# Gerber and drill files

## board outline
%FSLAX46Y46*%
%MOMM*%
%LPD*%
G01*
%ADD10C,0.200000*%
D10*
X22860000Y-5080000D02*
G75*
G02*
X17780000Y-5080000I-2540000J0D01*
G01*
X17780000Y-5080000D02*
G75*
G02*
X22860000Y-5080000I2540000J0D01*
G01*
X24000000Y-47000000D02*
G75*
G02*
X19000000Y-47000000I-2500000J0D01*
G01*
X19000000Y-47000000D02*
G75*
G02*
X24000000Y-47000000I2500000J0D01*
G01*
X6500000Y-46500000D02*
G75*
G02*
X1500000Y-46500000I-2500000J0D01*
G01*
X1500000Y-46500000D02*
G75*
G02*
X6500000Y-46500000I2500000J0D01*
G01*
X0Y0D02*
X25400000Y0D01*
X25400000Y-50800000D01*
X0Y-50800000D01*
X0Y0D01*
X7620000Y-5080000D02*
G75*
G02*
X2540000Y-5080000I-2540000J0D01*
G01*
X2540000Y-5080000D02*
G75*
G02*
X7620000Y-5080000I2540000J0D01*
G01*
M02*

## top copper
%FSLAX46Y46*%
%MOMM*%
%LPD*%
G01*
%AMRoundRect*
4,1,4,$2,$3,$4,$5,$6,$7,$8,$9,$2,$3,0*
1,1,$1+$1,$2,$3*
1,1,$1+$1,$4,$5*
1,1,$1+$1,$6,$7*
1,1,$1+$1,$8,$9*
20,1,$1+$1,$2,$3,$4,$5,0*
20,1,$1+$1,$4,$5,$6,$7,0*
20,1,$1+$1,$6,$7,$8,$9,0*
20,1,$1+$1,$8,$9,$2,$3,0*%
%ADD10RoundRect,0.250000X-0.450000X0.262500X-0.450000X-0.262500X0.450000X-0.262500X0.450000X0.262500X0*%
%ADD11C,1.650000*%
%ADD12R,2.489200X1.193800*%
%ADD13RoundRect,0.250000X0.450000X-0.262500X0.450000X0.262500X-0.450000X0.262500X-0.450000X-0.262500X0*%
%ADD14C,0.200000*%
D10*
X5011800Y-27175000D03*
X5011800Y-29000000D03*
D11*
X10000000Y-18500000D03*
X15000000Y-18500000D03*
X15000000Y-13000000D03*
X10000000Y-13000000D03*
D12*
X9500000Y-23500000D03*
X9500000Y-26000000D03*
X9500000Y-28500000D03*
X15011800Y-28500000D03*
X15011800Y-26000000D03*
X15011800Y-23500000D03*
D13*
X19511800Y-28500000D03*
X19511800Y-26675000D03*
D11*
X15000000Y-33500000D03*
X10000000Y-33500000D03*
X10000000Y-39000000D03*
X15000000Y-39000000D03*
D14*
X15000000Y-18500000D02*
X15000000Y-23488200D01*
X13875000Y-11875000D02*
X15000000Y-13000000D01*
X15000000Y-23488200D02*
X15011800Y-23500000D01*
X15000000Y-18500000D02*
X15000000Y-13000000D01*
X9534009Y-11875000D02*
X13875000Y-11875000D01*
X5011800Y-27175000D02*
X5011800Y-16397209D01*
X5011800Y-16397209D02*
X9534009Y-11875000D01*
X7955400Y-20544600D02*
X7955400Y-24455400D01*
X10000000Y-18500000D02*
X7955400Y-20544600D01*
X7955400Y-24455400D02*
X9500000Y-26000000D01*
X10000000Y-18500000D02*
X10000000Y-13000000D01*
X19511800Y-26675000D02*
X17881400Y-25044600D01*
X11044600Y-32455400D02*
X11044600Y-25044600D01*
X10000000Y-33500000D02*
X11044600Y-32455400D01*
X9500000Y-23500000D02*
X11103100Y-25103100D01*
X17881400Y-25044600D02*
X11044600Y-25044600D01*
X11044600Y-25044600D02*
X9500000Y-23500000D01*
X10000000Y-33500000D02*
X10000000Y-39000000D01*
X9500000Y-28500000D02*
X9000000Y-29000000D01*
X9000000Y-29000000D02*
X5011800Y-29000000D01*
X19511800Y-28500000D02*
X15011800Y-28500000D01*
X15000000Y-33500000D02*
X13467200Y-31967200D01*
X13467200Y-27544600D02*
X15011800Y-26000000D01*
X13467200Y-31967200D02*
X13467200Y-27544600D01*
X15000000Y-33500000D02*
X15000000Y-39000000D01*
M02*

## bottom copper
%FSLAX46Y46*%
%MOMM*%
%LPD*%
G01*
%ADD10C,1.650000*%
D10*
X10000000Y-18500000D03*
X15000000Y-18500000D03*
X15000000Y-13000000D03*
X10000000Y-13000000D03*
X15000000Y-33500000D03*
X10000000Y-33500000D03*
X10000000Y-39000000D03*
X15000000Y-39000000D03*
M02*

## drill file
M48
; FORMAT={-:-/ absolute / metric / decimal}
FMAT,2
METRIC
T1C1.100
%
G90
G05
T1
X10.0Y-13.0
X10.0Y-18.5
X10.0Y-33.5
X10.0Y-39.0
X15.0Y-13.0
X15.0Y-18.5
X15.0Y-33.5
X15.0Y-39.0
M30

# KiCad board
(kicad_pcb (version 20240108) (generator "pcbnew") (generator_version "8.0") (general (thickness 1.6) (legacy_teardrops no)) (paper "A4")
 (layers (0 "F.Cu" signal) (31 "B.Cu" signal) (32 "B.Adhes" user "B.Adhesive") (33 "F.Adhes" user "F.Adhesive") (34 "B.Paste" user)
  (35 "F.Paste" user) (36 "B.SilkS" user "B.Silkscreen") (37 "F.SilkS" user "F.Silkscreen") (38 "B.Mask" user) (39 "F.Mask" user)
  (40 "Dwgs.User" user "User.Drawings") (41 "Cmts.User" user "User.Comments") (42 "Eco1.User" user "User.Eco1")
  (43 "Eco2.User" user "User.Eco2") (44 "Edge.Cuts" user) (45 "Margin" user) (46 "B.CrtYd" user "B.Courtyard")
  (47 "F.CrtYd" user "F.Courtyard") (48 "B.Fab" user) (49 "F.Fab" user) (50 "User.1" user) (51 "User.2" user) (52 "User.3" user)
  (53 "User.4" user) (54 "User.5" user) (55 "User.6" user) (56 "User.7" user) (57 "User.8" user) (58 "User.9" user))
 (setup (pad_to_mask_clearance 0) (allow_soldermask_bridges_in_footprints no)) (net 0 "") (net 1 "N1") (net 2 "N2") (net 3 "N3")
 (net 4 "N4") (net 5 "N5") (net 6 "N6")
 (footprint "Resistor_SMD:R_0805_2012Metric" (layer "F.Cu") (at 5.0118 28.0875 -90)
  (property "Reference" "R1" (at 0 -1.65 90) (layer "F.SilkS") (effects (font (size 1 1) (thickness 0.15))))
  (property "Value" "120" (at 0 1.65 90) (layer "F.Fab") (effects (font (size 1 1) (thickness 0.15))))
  (pad "1" smd roundrect (at -0.9125 0 270) (size 1.025 1.4) (layers "F.Cu" "F.Paste" "F.Mask") (roundrect_rratio 0.243902) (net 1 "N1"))
  (pad "2" smd roundrect (at 0.9125 0 270) (size 1.025 1.4) (layers "F.Cu" "F.Paste" "F.Mask") (roundrect_rratio 0.243902) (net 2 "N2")))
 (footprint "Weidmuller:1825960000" (layer "F.Cu") (at 10 18.5)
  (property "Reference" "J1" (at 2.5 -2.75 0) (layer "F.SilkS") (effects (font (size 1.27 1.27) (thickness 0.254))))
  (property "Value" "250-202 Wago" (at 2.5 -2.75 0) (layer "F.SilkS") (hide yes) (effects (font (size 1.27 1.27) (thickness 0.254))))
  (pad "1" thru_hole circle (at 0 0) (size 1.65 1.65) (drill 1.1) (layers "*.Cu" "*.Mask") (remove_unused_layers no) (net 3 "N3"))
  (pad "2" thru_hole circle (at 5 0) (size 1.65 1.65) (drill 1.1) (layers "*.Cu" "*.Mask") (remove_unused_layers no) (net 1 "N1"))
  (pad "3" thru_hole circle (at 5 -5.5) (size 1.65 1.65) (drill 1.1) (layers "*.Cu" "*.Mask") (remove_unused_layers no) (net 1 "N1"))
  (pad "4" thru_hole circle (at 0 -5.5) (size 1.65 1.65) (drill 1.1) (layers "*.Cu" "*.Mask") (remove_unused_layers no) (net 3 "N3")))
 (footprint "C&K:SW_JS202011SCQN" (layer "F.Cu") (at 12.2559 26)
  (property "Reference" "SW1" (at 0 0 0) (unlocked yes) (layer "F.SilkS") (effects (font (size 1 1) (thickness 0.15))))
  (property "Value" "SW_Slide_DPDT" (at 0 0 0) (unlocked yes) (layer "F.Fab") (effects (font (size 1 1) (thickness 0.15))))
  (pad "1" smd rect (at -2.7559 -2.5) (size 2.4892 1.1938) (layers "F.Cu" "F.Paste" "F.Mask") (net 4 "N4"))
  (pad "2" smd rect (at -2.7559 0) (size 2.4892 1.1938) (layers "F.Cu" "F.Paste" "F.Mask") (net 3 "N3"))
  (pad "3" smd rect (at -2.7559 2.5) (size 2.4892 1.1938) (layers "F.Cu" "F.Paste" "F.Mask") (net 2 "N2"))
  (pad "4" smd rect (at 2.7559 2.5) (size 2.4892 1.1938) (layers "F.Cu" "F.Paste" "F.Mask") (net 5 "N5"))
  (pad "5" smd rect (at 2.7559 0) (size 2.4892 1.1938) (layers "F.Cu" "F.Paste" "F.Mask") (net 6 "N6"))
  (pad "6" smd rect (at 2.7559 -2.5) (size 2.4892 1.1938) (layers "F.Cu" "F.Paste" "F.Mask") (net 1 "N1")))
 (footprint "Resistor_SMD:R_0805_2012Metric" (layer "F.Cu") (at 19.5118 27.5875 90)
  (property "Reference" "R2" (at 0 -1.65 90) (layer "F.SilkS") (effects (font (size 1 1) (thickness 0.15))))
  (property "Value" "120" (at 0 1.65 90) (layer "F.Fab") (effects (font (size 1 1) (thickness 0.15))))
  (pad "1" smd roundrect (at -0.9125 0 90) (size 1.025 1.4) (layers "F.Cu" "F.Paste" "F.Mask") (roundrect_rratio 0.243902) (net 5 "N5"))
  (pad "2" smd roundrect (at 0.9125 0 90) (size 1.025 1.4) (layers "F.Cu" "F.Paste" "F.Mask") (roundrect_rratio 0.243902) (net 4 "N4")))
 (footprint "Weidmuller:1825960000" (layer "F.Cu") (at 15 33.5 180)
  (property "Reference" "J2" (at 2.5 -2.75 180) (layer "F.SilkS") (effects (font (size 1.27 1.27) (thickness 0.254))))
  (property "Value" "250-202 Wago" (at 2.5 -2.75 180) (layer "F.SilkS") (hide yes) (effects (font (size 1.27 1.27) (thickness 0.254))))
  (pad "1" thru_hole circle (at 0 0 180) (size 1.65 1.65) (drill 1.1) (layers "*.Cu" "*.Mask") (remove_unused_layers no) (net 6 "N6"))
  (pad "2" thru_hole circle (at 5 0 180) (size 1.65 1.65) (drill 1.1) (layers "*.Cu" "*.Mask") (remove_unused_layers no) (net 4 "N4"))
  (pad "3" thru_hole circle (at 5 -5.5 180) (size 1.65 1.65) (drill 1.1) (layers "*.Cu" "*.Mask") (remove_unused_layers no) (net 4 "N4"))
  (pad "4" thru_hole circle (at 0 -5.5 180) (size 1.65 1.65) (drill 1.1) (layers "*.Cu" "*.Mask") (remove_unused_layers no) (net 6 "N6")))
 (gr_circle (center 20.32 5.08) (end 22.86 5.08) (stroke (width 0.2) (type default)) (fill none) (layer "Edge.Cuts"))
 (gr_circle (center 21.5 47) (end 24 47) (stroke (width 0.2) (type default)) (fill none) (layer "Edge.Cuts"))
 (gr_circle (center 4 46.5) (end 6.5 46.5) (stroke (width 0.2) (type default)) (fill none) (layer "Edge.Cuts"))
 (gr_rect (start 0 0) (end 25.4 50.8) (stroke (width 0.2) (type default)) (fill none) (layer "Edge.Cuts"))
 (gr_circle (center 5.08 5.08) (end 7.62 5.08) (stroke (width 0.2) (type default)) (fill none) (layer "Edge.Cuts"))
 (segment (start 15 18.5) (end 15 23.4882) (width 0.2) (layer "F.Cu") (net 1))
 (segment (start 13.875 11.875) (end 15 13) (width 0.2) (layer "F.Cu") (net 1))
 (segment (start 15 23.4882) (end 15.0118 23.5) (width 0.2) (layer "F.Cu") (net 1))
 (segment (start 15 18.5) (end 15 13) (width 0.2) (layer "F.Cu") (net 1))
 (segment (start 9.534009 11.875) (end 13.875 11.875) (width 0.2) (layer "F.Cu") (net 1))
 (segment (start 5.0118 27.175) (end 5.0118 16.397209) (width 0.2) (layer "F.Cu") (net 1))
 (segment (start 5.0118 16.397209) (end 9.534009 11.875) (width 0.2) (layer "F.Cu") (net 1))
 (segment (start 7.9554 20.5446) (end 7.9554 24.4554) (width 0.2) (layer "F.Cu") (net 3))
 (segment (start 10 18.5) (end 7.9554 20.5446) (width 0.2) (layer "F.Cu") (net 3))
 (segment (start 7.9554 24.4554) (end 9.5 26) (width 0.2) (layer "F.Cu") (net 3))
 (segment (start 10 18.5) (end 10 13) (width 0.2) (layer "F.Cu") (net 3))
 (segment (start 19.5118 26.675) (end 17.8814 25.0446) (width 0.2) (layer "F.Cu") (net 4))
 (segment (start 11.0446 32.4554) (end 11.0446 25.0446) (width 0.2) (layer "F.Cu") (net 4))
 (segment (start 10 33.5) (end 11.0446 32.4554) (width 0.2) (layer "F.Cu") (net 4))
 (segment (start 9.5 23.5) (end 11.1031 25.1031) (width 0.2) (layer "F.Cu") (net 4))
 (segment (start 17.8814 25.0446) (end 11.0446 25.0446) (width 0.2) (layer "F.Cu") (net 4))
 (segment (start 11.0446 25.0446) (end 9.5 23.5) (width 0.2) (layer "F.Cu") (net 4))
 (segment (start 10 33.5) (end 10 39) (width 0.2) (layer "F.Cu") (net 4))
 (segment (start 9.5 28.5) (end 9 29) (width 0.2) (layer "F.Cu") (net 2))
 (segment (start 9 29) (end 5.0118 29) (width 0.2) (layer "F.Cu") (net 2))
 (segment (start 19.5118 28.5) (end 15.0118 28.5) (width 0.2) (layer "F.Cu") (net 5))
 (segment (start 15 33.5) (end 13.4672 31.9672) (width 0.2) (layer "F.Cu") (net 6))
 (segment (start 13.4672 27.5446) (end 15.0118 26) (width 0.2) (layer "F.Cu") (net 6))
 (segment (start 13.4672 31.9672) (end 13.4672 27.5446) (width 0.2) (layer "F.Cu") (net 6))
 (segment (start 15 33.5) (end 15 39) (width 0.2) (layer "F.Cu") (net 6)))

